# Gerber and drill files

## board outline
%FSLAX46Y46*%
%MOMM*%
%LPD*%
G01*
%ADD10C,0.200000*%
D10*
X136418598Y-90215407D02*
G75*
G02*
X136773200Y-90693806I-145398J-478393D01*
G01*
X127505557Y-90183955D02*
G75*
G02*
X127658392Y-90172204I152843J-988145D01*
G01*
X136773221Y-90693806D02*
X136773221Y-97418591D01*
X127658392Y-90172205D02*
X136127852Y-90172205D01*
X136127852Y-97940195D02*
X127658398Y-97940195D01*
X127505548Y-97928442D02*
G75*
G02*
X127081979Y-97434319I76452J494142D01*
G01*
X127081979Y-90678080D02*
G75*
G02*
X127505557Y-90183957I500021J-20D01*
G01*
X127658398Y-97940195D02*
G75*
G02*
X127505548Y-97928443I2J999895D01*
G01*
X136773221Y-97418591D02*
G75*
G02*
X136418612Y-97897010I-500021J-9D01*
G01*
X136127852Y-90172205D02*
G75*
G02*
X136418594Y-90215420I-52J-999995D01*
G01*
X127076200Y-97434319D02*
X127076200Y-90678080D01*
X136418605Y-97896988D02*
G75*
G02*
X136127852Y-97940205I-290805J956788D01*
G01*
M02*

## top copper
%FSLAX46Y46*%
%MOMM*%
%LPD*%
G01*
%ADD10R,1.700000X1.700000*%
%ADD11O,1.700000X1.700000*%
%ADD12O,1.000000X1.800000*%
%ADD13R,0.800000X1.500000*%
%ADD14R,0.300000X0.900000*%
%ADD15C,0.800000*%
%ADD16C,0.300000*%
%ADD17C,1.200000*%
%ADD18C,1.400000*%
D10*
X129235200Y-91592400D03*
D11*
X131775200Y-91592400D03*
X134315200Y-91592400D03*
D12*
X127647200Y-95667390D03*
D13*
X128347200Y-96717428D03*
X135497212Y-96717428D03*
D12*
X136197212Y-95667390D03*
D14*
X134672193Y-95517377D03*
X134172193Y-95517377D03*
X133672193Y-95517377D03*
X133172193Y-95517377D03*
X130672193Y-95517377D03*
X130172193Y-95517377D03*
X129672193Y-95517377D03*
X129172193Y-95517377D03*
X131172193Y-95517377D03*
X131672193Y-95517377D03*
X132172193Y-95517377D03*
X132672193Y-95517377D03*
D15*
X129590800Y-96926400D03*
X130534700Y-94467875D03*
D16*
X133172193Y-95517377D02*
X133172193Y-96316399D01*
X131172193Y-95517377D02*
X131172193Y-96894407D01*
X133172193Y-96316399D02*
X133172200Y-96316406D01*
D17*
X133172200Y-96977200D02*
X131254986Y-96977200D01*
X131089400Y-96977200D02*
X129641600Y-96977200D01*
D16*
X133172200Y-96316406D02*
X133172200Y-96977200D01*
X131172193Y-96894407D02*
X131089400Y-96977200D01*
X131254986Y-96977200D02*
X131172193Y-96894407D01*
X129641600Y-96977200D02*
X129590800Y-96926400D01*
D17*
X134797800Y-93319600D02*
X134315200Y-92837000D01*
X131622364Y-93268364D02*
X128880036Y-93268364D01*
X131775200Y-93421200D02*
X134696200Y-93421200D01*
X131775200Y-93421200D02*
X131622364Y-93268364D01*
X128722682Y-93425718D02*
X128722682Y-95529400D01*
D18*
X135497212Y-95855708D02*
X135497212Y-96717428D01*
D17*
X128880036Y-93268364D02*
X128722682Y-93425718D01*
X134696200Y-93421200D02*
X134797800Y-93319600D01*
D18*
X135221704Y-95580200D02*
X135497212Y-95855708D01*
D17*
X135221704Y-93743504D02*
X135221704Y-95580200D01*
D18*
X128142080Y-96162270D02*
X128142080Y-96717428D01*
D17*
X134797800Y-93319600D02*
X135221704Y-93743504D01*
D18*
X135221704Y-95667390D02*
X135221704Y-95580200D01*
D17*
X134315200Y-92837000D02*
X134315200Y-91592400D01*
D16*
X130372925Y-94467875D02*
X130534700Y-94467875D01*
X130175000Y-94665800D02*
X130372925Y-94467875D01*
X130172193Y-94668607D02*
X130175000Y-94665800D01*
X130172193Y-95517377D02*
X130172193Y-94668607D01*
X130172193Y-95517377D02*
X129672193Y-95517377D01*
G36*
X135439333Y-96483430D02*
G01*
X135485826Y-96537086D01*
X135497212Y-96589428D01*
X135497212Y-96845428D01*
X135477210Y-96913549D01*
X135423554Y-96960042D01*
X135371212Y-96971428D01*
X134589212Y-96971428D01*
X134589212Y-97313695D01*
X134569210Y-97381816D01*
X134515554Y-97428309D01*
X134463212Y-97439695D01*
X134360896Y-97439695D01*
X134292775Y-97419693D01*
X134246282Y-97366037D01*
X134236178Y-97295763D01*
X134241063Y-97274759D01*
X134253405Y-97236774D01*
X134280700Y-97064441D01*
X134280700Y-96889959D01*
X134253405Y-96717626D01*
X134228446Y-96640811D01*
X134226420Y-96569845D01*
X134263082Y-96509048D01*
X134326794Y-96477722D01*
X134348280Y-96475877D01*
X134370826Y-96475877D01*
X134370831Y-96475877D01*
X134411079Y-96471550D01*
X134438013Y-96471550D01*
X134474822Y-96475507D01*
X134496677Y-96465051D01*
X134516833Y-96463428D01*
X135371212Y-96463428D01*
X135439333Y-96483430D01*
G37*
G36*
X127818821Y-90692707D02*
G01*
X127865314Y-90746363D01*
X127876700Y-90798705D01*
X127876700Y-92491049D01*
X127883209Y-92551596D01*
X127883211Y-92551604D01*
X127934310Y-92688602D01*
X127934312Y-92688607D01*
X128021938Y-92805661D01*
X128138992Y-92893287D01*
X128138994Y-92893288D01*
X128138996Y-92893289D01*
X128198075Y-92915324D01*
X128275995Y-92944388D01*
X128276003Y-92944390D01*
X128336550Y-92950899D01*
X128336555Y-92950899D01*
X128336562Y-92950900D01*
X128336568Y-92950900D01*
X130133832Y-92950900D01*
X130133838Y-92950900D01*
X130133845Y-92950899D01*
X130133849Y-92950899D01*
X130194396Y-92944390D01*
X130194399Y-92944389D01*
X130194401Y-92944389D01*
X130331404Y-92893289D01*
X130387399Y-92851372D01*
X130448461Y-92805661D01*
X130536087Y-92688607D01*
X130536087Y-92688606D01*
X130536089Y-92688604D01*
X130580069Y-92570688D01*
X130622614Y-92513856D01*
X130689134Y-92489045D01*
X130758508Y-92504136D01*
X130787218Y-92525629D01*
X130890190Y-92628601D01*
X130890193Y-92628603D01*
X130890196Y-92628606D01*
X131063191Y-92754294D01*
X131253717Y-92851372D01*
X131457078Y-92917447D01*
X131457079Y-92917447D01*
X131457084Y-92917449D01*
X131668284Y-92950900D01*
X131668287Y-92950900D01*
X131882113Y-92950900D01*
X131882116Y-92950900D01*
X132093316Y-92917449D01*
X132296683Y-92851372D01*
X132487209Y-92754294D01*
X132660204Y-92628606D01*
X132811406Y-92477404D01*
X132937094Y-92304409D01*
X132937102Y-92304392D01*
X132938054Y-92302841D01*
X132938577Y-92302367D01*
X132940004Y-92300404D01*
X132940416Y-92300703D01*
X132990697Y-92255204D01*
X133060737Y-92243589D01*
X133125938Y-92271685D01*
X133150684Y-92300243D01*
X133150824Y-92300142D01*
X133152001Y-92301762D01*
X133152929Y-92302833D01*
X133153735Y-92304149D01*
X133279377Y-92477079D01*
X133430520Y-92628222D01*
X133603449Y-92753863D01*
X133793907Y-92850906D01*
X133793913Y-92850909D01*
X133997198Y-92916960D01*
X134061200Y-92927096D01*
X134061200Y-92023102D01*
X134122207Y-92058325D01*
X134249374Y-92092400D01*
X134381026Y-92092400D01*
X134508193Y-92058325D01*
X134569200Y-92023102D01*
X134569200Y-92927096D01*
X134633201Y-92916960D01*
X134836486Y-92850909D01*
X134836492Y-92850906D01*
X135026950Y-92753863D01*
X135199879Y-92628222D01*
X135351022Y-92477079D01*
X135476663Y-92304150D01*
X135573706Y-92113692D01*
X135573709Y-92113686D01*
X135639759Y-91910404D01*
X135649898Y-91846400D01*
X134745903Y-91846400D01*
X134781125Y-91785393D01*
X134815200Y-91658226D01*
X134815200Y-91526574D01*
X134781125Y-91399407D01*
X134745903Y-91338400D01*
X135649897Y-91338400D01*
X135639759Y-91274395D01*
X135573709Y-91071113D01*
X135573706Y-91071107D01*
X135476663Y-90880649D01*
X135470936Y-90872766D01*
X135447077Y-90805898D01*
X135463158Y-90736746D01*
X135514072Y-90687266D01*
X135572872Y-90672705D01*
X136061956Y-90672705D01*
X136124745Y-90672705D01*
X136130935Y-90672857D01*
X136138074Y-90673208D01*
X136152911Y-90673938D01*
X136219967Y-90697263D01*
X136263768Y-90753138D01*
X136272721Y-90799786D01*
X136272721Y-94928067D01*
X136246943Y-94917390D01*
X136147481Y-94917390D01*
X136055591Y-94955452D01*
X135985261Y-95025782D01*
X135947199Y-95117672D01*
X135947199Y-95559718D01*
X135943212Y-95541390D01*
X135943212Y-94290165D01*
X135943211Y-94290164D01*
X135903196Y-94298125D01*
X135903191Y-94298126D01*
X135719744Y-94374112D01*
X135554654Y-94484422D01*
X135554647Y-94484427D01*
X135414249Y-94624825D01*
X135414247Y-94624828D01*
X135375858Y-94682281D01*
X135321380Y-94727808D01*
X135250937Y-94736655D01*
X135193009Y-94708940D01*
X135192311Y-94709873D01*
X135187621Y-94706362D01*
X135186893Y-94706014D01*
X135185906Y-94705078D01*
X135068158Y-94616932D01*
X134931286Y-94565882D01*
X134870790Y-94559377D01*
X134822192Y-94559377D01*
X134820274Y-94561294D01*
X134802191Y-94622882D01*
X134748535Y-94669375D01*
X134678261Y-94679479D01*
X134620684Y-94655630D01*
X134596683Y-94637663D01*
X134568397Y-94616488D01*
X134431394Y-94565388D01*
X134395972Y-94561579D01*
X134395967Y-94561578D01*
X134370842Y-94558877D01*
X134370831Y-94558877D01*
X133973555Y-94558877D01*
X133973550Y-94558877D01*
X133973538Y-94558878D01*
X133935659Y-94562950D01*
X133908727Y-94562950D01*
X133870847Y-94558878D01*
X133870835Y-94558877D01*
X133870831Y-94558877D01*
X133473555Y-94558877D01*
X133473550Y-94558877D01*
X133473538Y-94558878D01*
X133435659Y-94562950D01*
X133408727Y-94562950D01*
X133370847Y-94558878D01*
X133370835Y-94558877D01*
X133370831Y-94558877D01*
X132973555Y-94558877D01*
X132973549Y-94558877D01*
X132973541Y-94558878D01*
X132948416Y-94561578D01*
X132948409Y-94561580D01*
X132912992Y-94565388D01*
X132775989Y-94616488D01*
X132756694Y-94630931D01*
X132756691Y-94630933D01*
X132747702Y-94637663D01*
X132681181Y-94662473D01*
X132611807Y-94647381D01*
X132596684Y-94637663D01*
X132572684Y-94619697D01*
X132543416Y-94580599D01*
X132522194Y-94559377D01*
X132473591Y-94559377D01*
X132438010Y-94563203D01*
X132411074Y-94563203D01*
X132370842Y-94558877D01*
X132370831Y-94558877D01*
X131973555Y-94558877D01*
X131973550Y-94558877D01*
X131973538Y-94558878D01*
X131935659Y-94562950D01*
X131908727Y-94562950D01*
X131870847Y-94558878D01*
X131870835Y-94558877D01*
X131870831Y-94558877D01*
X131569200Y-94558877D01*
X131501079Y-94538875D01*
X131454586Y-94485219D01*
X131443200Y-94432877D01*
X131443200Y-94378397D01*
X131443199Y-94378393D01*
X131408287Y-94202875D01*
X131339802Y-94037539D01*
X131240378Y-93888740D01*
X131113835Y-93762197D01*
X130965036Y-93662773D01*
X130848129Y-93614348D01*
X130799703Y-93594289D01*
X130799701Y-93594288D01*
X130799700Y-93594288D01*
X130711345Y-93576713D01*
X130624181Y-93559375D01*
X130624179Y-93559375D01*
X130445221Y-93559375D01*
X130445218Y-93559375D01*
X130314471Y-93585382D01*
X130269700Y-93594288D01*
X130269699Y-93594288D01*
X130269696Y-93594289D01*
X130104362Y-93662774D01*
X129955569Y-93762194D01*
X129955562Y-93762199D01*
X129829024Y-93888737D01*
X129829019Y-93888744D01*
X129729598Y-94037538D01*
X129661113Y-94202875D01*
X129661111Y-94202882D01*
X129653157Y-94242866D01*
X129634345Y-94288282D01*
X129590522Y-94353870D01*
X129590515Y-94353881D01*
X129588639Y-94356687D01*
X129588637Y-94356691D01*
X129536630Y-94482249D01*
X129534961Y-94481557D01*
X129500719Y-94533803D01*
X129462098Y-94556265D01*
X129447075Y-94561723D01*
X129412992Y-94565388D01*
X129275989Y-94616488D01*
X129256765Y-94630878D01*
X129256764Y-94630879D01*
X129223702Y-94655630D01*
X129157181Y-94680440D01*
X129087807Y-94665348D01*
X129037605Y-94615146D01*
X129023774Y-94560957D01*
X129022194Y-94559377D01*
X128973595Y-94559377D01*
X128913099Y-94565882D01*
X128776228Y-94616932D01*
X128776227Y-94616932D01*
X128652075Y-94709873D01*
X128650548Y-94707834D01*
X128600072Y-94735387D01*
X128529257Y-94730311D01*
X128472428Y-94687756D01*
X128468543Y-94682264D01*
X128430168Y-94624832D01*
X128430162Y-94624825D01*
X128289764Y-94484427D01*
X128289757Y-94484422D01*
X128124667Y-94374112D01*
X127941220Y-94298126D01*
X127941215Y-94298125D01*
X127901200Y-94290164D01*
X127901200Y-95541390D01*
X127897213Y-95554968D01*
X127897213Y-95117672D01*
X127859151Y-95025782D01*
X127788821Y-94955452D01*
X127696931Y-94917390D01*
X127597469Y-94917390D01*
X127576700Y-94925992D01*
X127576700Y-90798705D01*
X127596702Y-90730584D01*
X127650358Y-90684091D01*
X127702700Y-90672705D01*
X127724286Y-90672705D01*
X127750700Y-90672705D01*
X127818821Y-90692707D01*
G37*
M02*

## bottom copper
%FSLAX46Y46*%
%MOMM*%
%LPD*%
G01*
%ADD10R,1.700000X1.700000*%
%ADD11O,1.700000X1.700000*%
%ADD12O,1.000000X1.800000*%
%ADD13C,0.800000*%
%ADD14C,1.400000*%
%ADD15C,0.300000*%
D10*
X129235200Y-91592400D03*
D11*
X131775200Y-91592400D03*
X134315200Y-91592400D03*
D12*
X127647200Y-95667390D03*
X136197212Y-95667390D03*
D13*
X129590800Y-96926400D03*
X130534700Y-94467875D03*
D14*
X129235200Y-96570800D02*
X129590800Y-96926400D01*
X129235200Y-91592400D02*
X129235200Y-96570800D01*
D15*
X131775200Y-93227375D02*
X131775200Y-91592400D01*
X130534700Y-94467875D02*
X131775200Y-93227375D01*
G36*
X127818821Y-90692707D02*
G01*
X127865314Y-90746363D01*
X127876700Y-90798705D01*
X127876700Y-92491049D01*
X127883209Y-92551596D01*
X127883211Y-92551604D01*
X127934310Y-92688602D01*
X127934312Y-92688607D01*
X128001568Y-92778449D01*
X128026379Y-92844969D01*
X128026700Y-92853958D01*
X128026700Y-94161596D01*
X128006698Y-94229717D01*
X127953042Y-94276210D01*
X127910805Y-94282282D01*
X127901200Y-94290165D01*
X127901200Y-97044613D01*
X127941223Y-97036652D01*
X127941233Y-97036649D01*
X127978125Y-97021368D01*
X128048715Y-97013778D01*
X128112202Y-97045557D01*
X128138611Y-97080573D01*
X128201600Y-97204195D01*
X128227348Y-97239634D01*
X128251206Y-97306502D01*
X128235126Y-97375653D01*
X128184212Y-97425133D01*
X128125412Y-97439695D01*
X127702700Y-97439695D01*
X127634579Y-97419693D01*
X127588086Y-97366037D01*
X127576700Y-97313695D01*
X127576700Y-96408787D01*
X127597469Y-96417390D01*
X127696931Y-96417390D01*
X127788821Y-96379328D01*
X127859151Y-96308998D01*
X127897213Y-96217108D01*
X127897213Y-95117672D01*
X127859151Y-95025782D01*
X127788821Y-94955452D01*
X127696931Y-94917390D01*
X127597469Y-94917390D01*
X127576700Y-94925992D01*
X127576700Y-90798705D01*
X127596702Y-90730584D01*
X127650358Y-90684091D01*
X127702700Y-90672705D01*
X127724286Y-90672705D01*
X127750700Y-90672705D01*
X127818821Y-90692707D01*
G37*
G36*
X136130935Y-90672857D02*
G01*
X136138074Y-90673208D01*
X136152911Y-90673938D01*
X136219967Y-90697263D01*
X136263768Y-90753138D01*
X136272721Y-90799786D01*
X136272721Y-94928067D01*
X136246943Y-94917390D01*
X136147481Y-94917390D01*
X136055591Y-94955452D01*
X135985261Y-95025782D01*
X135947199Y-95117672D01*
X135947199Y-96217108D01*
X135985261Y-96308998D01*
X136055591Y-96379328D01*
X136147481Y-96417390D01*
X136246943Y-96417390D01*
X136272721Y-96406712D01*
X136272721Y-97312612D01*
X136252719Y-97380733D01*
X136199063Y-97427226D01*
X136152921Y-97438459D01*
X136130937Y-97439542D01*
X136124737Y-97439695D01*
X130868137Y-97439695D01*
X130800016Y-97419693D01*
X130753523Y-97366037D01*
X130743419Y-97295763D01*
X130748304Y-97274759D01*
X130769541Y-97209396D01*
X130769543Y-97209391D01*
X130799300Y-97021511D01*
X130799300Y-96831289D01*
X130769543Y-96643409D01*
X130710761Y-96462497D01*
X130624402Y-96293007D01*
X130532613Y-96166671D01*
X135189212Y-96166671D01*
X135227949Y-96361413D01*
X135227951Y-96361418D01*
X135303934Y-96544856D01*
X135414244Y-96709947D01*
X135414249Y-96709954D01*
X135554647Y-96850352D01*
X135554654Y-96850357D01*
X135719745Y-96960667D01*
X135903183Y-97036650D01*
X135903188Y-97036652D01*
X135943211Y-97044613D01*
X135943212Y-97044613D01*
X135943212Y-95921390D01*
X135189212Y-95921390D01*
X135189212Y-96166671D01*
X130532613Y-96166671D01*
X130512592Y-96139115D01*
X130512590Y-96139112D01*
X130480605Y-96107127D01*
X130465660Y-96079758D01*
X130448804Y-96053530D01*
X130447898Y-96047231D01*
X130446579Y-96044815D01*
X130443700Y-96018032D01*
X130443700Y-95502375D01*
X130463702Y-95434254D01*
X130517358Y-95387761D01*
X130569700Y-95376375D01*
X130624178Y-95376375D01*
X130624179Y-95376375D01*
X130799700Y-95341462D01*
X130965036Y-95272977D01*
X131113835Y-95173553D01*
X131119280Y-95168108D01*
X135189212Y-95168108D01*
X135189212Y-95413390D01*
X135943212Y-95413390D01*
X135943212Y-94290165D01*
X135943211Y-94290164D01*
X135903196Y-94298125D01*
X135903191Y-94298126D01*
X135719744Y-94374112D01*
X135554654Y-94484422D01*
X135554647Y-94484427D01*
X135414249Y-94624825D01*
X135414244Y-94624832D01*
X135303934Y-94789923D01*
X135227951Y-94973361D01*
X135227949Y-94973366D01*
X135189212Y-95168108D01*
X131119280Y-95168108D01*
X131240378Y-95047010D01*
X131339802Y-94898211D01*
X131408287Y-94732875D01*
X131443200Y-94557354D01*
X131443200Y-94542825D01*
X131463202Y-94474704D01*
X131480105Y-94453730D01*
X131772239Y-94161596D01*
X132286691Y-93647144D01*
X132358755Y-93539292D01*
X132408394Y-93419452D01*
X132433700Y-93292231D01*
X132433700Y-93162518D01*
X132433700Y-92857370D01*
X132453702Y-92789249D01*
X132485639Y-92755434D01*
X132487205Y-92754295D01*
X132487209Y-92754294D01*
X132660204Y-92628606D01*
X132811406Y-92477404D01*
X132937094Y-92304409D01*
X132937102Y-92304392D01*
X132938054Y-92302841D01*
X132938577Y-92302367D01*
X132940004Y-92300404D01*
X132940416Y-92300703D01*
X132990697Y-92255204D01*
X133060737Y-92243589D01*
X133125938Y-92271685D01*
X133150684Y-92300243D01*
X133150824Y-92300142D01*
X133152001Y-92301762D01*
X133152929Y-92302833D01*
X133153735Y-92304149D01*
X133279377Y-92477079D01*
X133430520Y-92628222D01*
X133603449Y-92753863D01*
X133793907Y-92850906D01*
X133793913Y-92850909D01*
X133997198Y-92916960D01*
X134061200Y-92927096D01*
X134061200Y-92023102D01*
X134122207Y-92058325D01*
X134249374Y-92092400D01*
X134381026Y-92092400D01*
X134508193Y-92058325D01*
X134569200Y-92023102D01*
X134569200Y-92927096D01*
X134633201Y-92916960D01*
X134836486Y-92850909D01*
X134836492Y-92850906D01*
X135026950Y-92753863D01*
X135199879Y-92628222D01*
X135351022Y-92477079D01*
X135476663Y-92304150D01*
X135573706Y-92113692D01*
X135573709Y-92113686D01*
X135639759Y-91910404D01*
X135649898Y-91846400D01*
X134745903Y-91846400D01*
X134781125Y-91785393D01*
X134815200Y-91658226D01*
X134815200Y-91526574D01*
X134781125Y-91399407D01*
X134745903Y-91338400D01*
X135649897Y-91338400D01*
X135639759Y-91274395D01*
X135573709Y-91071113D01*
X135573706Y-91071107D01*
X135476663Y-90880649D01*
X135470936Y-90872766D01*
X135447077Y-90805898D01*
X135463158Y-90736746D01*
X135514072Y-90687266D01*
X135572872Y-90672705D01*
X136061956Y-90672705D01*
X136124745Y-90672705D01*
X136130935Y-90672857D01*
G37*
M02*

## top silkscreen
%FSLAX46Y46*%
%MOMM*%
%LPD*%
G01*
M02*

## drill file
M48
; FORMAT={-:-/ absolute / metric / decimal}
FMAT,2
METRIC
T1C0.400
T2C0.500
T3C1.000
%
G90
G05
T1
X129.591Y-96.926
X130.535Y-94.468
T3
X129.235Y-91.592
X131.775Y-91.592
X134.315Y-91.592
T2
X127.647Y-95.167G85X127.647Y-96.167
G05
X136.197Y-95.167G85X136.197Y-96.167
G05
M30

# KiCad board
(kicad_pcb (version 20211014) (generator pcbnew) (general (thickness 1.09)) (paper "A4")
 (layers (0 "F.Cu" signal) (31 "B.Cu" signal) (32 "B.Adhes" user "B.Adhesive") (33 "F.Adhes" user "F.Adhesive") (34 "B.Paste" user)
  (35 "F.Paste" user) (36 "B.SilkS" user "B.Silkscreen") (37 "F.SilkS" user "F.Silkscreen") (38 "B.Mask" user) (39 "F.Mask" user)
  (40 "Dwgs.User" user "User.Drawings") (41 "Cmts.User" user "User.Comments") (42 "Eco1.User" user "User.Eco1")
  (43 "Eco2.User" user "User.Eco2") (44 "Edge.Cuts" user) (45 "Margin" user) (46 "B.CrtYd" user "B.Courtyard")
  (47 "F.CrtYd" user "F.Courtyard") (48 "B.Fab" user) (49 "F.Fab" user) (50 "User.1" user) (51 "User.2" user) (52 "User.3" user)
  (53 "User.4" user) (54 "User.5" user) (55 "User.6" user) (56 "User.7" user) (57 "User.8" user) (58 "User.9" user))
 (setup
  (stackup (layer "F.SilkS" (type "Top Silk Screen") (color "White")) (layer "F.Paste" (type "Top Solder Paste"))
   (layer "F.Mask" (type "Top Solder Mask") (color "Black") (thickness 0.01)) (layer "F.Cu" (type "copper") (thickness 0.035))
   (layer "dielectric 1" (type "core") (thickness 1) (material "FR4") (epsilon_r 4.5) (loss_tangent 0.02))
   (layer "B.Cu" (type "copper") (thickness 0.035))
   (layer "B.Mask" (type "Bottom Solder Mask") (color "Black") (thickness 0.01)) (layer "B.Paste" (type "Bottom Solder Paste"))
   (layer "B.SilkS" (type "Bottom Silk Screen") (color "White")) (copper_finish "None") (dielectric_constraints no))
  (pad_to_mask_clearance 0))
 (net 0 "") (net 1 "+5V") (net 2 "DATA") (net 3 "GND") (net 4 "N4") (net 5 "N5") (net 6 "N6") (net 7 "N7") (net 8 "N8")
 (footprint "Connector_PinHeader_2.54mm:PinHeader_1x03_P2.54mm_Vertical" (layer "F.Cu") (at 129.2352 91.5924 90)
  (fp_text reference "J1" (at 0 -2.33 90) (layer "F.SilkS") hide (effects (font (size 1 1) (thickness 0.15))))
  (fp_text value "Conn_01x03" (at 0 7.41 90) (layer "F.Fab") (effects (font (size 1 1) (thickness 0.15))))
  (pad "1" thru_hole rect (at 0 0 90) (size 1.7 1.7) (drill 1) (layers *.Cu *.Mask) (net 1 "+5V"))
  (pad "2" thru_hole oval (at 0 2.54 90) (size 1.7 1.7) (drill 1) (layers *.Cu *.Mask) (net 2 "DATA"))
  (pad "3" thru_hole oval (at 0 5.08 90) (size 1.7 1.7) (drill 1) (layers *.Cu *.Mask) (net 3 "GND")))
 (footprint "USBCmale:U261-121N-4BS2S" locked (layer "F.Cu") (at 131.922206 101.959414)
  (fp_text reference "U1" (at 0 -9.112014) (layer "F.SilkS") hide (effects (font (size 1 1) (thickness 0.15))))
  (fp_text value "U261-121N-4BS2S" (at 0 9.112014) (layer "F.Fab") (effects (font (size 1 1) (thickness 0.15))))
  (pad "25" thru_hole oval locked (at -4.275006 -6.292024) (size 1 1.8) (drill oval 0.500025 1.5) (layers *.Cu *.Mask) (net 3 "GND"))
  (pad "25" smd rect locked (at -3.575006 -5.241986) (size 0.8 1.5) (layers "F.Cu" "F.Paste" "F.Mask") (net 3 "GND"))
  (pad "26" smd rect locked (at 3.575006 -5.241986) (size 0.8 1.5) (layers "F.Cu" "F.Paste" "F.Mask") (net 3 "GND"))
  (pad "26" thru_hole oval locked (at 4.275006 -6.292024) (size 1 1.8) (drill oval 0.500025 1.5) (layers *.Cu *.Mask) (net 3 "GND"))
  (pad "A1" smd rect locked (at 2.749987 -6.442037) (size 0.3 0.9) (layers "F.Cu" "F.Paste" "F.Mask") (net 3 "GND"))
  (pad "A2" smd rect locked (at 2.249987 -6.442037) (size 0.3 0.9) (layers "F.Cu" "F.Paste" "F.Mask") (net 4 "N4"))
  (pad "A3" smd rect locked (at 1.749987 -6.442037) (size 0.3 0.9) (layers "F.Cu" "F.Paste" "F.Mask") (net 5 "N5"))
  (pad "A4" smd rect locked (at 1.249987 -6.442037) (size 0.3 0.9) (layers "F.Cu" "F.Paste" "F.Mask") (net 1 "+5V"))
  (pad "A5" smd rect locked (at -1.250013 -6.442037) (size 0.3 0.9) (layers "F.Cu" "F.Paste" "F.Mask") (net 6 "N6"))
  (pad "A6" smd rect locked (at -1.750013 -6.442037) (size 0.3 0.9) (layers "F.Cu" "F.Paste" "F.Mask") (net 2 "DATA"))
  (pad "A7" smd rect locked (at -2.250013 -6.442037) (size 0.3 0.9) (layers "F.Cu" "F.Paste" "F.Mask") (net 2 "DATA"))
  (pad "A12" smd rect locked (at -2.750013 -6.442037) (size 0.3 0.9) (layers "F.Cu" "F.Paste" "F.Mask") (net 3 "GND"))
  (pad "B9" smd rect locked (at -0.750013 -6.442037) (size 0.3 0.9) (layers "F.Cu" "F.Paste" "F.Mask") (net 1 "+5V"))
  (pad "B10" smd rect locked (at -0.250013 -6.442037) (size 0.3 0.9) (layers "F.Cu" "F.Paste" "F.Mask") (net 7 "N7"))
  (pad "B11" smd rect locked (at 0.249987 -6.442037) (size 0.3 0.9) (layers "F.Cu" "F.Paste" "F.Mask") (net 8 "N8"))
  (pad "B12" smd rect locked (at 0.749987 -6.442037) (size 0.3 0.9) (layers "F.Cu" "F.Paste" "F.Mask") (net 3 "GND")))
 (gr_arc (start 136.418598 90.215407) (mid 136.674898 90.396055) (end 136.773221 90.693806) (layer "Edge.Cuts") (width 0.2))
 (gr_arc (start 127.505557 90.183955) (mid 127.581749 90.175147) (end 127.658392 90.172205) (layer "Edge.Cuts") (width 0.2))
 (gr_line (start 136.773221 90.693806) (end 136.773221 97.418591) (layer "Edge.Cuts") (width 0.2))
 (gr_line (start 127.658392 90.172205) (end 136.127852 90.172205) (layer "Edge.Cuts") (width 0.2))
 (gr_line (start 136.127852 97.940195) (end 127.658398 97.940195) (layer "Edge.Cuts") (width 0.2))
 (gr_arc (start 127.505548 97.928442) (mid 127.202363 97.75973) (end 127.081979 97.434319) (layer "Edge.Cuts") (width 0.2))
 (gr_arc (start 127.081979 90.67808) (mid 127.202366 90.352665) (end 127.505557 90.183955) (layer "Edge.Cuts") (width 0.2))
 (gr_arc (start 127.658398 97.940195) (mid 127.581747 97.937252) (end 127.505548 97.928442) (layer "Edge.Cuts") (width 0.2))
 (gr_arc (start 136.773221 97.418591) (mid 136.6749 97.716339) (end 136.418605 97.896988) (layer "Edge.Cuts") (width 0.2))
 (gr_arc (start 136.127852 90.172205) (mid 136.274821 90.183065) (end 136.418598 90.215407) (layer "Edge.Cuts") (width 0.2))
 (gr_line (start 127.0762 97.434319) (end 127.0762 90.67808) (layer "Edge.Cuts") (width 0.2))
 (gr_arc (start 136.418605 97.896988) (mid 136.274825 97.929333) (end 136.127852 97.940195) (layer "Edge.Cuts") (width 0.2))
 (segment (start 133.172193 95.517377) (end 133.172193 96.316399) (width 0.3) (layer "F.Cu") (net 1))
 (segment (start 131.172193 95.517377) (end 131.172193 96.894407) (width 0.3) (layer "F.Cu") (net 1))
 (segment (start 133.172193 96.316399) (end 133.1722 96.316406) (width 0.3) (layer "F.Cu") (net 1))
 (segment (start 133.1722 96.9772) (end 131.254986 96.9772) (width 1.2) (layer "F.Cu") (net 1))
 (segment (start 131.0894 96.9772) (end 129.6416 96.9772) (width 1.2) (layer "F.Cu") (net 1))
 (segment (start 133.1722 96.316406) (end 133.1722 96.9772) (width 0.3) (layer "F.Cu") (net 1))
 (segment (start 131.172193 96.894407) (end 131.0894 96.9772) (width 0.3) (layer "F.Cu") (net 1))
 (segment (start 131.254986 96.9772) (end 131.172193 96.894407) (width 0.3) (layer "F.Cu") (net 1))
 (segment (start 129.6416 96.9772) (end 129.5908 96.9264) (width 0.3) (layer "F.Cu") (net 1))
 (via (at 129.5908 96.9264) (size 0.8) (drill 0.4) (layers "F.Cu" "B.Cu") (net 1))
 (segment (start 129.2352 96.5708) (end 129.5908 96.9264) (width 1.4) (layer "B.Cu") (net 1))
 (segment (start 129.2352 91.5924) (end 129.2352 96.5708) (width 1.4) (layer "B.Cu") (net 1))
 (segment (start 134.7978 93.3196) (end 134.3152 92.837) (width 1.2) (layer "F.Cu") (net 3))
 (segment (start 131.622364 93.268364) (end 128.880036 93.268364) (width 1.2) (layer "F.Cu") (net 3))
 (segment (start 131.7752 93.4212) (end 134.6962 93.4212) (width 1.2) (layer "F.Cu") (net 3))
 (segment (start 131.7752 93.4212) (end 131.622364 93.268364) (width 1.2) (layer "F.Cu") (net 3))
 (segment (start 128.722682 93.425718) (end 128.722682 95.5294) (width 1.2) (layer "F.Cu") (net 3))
 (segment (start 135.497212 95.855708) (end 135.497212 96.717428) (width 1.4) (layer "F.Cu") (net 3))
 (segment (start 128.880036 93.268364) (end 128.722682 93.425718) (width 1.2) (layer "F.Cu") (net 3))
 (segment (start 134.6962 93.4212) (end 134.7978 93.3196) (width 1.2) (layer "F.Cu") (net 3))
 (segment (start 135.221704 95.5802) (end 135.497212 95.855708) (width 1.4) (layer "F.Cu") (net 3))
 (segment (start 135.221704 93.743504) (end 135.221704 95.5802) (width 1.2) (layer "F.Cu") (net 3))
 (segment (start 128.14208 96.16227) (end 128.14208 96.717428) (width 1.4) (layer "F.Cu") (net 3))
 (segment (start 134.7978 93.3196) (end 135.221704 93.743504) (width 1.2) (layer "F.Cu") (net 3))
 (segment (start 135.221704 95.66739) (end 135.221704 95.5802) (width 1.4) (layer "F.Cu") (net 3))
 (segment (start 134.3152 92.837) (end 134.3152 91.5924) (width 1.2) (layer "F.Cu") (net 3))
 (segment (start 130.372925 94.467875) (end 130.5347 94.467875) (width 0.3) (layer "F.Cu") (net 2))
 (segment (start 130.175 94.6658) (end 130.372925 94.467875) (width 0.3) (layer "F.Cu") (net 2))
 (segment (start 130.172193 94.668607) (end 130.175 94.6658) (width 0.3) (layer "F.Cu") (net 2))
 (segment (start 130.172193 95.517377) (end 130.172193 94.668607) (width 0.3) (layer "F.Cu") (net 2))
 (segment (start 130.172193 95.517377) (end 129.672193 95.517377) (width 0.3) (layer "F.Cu") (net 2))
 (via (at 130.5347 94.467875) (size 0.8) (drill 0.4) (layers "F.Cu" "B.Cu") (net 2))
 (segment (start 131.7752 93.227375) (end 131.7752 91.5924) (width 0.3) (layer "B.Cu") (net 2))
 (segment (start 130.5347 94.467875) (end 131.7752 93.227375) (width 0.3) (layer "B.Cu") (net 2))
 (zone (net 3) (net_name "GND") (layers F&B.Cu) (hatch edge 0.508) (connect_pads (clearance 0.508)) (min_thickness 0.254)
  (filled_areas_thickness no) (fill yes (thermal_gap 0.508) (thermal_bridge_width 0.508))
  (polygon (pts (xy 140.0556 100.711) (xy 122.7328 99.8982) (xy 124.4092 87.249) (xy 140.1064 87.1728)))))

